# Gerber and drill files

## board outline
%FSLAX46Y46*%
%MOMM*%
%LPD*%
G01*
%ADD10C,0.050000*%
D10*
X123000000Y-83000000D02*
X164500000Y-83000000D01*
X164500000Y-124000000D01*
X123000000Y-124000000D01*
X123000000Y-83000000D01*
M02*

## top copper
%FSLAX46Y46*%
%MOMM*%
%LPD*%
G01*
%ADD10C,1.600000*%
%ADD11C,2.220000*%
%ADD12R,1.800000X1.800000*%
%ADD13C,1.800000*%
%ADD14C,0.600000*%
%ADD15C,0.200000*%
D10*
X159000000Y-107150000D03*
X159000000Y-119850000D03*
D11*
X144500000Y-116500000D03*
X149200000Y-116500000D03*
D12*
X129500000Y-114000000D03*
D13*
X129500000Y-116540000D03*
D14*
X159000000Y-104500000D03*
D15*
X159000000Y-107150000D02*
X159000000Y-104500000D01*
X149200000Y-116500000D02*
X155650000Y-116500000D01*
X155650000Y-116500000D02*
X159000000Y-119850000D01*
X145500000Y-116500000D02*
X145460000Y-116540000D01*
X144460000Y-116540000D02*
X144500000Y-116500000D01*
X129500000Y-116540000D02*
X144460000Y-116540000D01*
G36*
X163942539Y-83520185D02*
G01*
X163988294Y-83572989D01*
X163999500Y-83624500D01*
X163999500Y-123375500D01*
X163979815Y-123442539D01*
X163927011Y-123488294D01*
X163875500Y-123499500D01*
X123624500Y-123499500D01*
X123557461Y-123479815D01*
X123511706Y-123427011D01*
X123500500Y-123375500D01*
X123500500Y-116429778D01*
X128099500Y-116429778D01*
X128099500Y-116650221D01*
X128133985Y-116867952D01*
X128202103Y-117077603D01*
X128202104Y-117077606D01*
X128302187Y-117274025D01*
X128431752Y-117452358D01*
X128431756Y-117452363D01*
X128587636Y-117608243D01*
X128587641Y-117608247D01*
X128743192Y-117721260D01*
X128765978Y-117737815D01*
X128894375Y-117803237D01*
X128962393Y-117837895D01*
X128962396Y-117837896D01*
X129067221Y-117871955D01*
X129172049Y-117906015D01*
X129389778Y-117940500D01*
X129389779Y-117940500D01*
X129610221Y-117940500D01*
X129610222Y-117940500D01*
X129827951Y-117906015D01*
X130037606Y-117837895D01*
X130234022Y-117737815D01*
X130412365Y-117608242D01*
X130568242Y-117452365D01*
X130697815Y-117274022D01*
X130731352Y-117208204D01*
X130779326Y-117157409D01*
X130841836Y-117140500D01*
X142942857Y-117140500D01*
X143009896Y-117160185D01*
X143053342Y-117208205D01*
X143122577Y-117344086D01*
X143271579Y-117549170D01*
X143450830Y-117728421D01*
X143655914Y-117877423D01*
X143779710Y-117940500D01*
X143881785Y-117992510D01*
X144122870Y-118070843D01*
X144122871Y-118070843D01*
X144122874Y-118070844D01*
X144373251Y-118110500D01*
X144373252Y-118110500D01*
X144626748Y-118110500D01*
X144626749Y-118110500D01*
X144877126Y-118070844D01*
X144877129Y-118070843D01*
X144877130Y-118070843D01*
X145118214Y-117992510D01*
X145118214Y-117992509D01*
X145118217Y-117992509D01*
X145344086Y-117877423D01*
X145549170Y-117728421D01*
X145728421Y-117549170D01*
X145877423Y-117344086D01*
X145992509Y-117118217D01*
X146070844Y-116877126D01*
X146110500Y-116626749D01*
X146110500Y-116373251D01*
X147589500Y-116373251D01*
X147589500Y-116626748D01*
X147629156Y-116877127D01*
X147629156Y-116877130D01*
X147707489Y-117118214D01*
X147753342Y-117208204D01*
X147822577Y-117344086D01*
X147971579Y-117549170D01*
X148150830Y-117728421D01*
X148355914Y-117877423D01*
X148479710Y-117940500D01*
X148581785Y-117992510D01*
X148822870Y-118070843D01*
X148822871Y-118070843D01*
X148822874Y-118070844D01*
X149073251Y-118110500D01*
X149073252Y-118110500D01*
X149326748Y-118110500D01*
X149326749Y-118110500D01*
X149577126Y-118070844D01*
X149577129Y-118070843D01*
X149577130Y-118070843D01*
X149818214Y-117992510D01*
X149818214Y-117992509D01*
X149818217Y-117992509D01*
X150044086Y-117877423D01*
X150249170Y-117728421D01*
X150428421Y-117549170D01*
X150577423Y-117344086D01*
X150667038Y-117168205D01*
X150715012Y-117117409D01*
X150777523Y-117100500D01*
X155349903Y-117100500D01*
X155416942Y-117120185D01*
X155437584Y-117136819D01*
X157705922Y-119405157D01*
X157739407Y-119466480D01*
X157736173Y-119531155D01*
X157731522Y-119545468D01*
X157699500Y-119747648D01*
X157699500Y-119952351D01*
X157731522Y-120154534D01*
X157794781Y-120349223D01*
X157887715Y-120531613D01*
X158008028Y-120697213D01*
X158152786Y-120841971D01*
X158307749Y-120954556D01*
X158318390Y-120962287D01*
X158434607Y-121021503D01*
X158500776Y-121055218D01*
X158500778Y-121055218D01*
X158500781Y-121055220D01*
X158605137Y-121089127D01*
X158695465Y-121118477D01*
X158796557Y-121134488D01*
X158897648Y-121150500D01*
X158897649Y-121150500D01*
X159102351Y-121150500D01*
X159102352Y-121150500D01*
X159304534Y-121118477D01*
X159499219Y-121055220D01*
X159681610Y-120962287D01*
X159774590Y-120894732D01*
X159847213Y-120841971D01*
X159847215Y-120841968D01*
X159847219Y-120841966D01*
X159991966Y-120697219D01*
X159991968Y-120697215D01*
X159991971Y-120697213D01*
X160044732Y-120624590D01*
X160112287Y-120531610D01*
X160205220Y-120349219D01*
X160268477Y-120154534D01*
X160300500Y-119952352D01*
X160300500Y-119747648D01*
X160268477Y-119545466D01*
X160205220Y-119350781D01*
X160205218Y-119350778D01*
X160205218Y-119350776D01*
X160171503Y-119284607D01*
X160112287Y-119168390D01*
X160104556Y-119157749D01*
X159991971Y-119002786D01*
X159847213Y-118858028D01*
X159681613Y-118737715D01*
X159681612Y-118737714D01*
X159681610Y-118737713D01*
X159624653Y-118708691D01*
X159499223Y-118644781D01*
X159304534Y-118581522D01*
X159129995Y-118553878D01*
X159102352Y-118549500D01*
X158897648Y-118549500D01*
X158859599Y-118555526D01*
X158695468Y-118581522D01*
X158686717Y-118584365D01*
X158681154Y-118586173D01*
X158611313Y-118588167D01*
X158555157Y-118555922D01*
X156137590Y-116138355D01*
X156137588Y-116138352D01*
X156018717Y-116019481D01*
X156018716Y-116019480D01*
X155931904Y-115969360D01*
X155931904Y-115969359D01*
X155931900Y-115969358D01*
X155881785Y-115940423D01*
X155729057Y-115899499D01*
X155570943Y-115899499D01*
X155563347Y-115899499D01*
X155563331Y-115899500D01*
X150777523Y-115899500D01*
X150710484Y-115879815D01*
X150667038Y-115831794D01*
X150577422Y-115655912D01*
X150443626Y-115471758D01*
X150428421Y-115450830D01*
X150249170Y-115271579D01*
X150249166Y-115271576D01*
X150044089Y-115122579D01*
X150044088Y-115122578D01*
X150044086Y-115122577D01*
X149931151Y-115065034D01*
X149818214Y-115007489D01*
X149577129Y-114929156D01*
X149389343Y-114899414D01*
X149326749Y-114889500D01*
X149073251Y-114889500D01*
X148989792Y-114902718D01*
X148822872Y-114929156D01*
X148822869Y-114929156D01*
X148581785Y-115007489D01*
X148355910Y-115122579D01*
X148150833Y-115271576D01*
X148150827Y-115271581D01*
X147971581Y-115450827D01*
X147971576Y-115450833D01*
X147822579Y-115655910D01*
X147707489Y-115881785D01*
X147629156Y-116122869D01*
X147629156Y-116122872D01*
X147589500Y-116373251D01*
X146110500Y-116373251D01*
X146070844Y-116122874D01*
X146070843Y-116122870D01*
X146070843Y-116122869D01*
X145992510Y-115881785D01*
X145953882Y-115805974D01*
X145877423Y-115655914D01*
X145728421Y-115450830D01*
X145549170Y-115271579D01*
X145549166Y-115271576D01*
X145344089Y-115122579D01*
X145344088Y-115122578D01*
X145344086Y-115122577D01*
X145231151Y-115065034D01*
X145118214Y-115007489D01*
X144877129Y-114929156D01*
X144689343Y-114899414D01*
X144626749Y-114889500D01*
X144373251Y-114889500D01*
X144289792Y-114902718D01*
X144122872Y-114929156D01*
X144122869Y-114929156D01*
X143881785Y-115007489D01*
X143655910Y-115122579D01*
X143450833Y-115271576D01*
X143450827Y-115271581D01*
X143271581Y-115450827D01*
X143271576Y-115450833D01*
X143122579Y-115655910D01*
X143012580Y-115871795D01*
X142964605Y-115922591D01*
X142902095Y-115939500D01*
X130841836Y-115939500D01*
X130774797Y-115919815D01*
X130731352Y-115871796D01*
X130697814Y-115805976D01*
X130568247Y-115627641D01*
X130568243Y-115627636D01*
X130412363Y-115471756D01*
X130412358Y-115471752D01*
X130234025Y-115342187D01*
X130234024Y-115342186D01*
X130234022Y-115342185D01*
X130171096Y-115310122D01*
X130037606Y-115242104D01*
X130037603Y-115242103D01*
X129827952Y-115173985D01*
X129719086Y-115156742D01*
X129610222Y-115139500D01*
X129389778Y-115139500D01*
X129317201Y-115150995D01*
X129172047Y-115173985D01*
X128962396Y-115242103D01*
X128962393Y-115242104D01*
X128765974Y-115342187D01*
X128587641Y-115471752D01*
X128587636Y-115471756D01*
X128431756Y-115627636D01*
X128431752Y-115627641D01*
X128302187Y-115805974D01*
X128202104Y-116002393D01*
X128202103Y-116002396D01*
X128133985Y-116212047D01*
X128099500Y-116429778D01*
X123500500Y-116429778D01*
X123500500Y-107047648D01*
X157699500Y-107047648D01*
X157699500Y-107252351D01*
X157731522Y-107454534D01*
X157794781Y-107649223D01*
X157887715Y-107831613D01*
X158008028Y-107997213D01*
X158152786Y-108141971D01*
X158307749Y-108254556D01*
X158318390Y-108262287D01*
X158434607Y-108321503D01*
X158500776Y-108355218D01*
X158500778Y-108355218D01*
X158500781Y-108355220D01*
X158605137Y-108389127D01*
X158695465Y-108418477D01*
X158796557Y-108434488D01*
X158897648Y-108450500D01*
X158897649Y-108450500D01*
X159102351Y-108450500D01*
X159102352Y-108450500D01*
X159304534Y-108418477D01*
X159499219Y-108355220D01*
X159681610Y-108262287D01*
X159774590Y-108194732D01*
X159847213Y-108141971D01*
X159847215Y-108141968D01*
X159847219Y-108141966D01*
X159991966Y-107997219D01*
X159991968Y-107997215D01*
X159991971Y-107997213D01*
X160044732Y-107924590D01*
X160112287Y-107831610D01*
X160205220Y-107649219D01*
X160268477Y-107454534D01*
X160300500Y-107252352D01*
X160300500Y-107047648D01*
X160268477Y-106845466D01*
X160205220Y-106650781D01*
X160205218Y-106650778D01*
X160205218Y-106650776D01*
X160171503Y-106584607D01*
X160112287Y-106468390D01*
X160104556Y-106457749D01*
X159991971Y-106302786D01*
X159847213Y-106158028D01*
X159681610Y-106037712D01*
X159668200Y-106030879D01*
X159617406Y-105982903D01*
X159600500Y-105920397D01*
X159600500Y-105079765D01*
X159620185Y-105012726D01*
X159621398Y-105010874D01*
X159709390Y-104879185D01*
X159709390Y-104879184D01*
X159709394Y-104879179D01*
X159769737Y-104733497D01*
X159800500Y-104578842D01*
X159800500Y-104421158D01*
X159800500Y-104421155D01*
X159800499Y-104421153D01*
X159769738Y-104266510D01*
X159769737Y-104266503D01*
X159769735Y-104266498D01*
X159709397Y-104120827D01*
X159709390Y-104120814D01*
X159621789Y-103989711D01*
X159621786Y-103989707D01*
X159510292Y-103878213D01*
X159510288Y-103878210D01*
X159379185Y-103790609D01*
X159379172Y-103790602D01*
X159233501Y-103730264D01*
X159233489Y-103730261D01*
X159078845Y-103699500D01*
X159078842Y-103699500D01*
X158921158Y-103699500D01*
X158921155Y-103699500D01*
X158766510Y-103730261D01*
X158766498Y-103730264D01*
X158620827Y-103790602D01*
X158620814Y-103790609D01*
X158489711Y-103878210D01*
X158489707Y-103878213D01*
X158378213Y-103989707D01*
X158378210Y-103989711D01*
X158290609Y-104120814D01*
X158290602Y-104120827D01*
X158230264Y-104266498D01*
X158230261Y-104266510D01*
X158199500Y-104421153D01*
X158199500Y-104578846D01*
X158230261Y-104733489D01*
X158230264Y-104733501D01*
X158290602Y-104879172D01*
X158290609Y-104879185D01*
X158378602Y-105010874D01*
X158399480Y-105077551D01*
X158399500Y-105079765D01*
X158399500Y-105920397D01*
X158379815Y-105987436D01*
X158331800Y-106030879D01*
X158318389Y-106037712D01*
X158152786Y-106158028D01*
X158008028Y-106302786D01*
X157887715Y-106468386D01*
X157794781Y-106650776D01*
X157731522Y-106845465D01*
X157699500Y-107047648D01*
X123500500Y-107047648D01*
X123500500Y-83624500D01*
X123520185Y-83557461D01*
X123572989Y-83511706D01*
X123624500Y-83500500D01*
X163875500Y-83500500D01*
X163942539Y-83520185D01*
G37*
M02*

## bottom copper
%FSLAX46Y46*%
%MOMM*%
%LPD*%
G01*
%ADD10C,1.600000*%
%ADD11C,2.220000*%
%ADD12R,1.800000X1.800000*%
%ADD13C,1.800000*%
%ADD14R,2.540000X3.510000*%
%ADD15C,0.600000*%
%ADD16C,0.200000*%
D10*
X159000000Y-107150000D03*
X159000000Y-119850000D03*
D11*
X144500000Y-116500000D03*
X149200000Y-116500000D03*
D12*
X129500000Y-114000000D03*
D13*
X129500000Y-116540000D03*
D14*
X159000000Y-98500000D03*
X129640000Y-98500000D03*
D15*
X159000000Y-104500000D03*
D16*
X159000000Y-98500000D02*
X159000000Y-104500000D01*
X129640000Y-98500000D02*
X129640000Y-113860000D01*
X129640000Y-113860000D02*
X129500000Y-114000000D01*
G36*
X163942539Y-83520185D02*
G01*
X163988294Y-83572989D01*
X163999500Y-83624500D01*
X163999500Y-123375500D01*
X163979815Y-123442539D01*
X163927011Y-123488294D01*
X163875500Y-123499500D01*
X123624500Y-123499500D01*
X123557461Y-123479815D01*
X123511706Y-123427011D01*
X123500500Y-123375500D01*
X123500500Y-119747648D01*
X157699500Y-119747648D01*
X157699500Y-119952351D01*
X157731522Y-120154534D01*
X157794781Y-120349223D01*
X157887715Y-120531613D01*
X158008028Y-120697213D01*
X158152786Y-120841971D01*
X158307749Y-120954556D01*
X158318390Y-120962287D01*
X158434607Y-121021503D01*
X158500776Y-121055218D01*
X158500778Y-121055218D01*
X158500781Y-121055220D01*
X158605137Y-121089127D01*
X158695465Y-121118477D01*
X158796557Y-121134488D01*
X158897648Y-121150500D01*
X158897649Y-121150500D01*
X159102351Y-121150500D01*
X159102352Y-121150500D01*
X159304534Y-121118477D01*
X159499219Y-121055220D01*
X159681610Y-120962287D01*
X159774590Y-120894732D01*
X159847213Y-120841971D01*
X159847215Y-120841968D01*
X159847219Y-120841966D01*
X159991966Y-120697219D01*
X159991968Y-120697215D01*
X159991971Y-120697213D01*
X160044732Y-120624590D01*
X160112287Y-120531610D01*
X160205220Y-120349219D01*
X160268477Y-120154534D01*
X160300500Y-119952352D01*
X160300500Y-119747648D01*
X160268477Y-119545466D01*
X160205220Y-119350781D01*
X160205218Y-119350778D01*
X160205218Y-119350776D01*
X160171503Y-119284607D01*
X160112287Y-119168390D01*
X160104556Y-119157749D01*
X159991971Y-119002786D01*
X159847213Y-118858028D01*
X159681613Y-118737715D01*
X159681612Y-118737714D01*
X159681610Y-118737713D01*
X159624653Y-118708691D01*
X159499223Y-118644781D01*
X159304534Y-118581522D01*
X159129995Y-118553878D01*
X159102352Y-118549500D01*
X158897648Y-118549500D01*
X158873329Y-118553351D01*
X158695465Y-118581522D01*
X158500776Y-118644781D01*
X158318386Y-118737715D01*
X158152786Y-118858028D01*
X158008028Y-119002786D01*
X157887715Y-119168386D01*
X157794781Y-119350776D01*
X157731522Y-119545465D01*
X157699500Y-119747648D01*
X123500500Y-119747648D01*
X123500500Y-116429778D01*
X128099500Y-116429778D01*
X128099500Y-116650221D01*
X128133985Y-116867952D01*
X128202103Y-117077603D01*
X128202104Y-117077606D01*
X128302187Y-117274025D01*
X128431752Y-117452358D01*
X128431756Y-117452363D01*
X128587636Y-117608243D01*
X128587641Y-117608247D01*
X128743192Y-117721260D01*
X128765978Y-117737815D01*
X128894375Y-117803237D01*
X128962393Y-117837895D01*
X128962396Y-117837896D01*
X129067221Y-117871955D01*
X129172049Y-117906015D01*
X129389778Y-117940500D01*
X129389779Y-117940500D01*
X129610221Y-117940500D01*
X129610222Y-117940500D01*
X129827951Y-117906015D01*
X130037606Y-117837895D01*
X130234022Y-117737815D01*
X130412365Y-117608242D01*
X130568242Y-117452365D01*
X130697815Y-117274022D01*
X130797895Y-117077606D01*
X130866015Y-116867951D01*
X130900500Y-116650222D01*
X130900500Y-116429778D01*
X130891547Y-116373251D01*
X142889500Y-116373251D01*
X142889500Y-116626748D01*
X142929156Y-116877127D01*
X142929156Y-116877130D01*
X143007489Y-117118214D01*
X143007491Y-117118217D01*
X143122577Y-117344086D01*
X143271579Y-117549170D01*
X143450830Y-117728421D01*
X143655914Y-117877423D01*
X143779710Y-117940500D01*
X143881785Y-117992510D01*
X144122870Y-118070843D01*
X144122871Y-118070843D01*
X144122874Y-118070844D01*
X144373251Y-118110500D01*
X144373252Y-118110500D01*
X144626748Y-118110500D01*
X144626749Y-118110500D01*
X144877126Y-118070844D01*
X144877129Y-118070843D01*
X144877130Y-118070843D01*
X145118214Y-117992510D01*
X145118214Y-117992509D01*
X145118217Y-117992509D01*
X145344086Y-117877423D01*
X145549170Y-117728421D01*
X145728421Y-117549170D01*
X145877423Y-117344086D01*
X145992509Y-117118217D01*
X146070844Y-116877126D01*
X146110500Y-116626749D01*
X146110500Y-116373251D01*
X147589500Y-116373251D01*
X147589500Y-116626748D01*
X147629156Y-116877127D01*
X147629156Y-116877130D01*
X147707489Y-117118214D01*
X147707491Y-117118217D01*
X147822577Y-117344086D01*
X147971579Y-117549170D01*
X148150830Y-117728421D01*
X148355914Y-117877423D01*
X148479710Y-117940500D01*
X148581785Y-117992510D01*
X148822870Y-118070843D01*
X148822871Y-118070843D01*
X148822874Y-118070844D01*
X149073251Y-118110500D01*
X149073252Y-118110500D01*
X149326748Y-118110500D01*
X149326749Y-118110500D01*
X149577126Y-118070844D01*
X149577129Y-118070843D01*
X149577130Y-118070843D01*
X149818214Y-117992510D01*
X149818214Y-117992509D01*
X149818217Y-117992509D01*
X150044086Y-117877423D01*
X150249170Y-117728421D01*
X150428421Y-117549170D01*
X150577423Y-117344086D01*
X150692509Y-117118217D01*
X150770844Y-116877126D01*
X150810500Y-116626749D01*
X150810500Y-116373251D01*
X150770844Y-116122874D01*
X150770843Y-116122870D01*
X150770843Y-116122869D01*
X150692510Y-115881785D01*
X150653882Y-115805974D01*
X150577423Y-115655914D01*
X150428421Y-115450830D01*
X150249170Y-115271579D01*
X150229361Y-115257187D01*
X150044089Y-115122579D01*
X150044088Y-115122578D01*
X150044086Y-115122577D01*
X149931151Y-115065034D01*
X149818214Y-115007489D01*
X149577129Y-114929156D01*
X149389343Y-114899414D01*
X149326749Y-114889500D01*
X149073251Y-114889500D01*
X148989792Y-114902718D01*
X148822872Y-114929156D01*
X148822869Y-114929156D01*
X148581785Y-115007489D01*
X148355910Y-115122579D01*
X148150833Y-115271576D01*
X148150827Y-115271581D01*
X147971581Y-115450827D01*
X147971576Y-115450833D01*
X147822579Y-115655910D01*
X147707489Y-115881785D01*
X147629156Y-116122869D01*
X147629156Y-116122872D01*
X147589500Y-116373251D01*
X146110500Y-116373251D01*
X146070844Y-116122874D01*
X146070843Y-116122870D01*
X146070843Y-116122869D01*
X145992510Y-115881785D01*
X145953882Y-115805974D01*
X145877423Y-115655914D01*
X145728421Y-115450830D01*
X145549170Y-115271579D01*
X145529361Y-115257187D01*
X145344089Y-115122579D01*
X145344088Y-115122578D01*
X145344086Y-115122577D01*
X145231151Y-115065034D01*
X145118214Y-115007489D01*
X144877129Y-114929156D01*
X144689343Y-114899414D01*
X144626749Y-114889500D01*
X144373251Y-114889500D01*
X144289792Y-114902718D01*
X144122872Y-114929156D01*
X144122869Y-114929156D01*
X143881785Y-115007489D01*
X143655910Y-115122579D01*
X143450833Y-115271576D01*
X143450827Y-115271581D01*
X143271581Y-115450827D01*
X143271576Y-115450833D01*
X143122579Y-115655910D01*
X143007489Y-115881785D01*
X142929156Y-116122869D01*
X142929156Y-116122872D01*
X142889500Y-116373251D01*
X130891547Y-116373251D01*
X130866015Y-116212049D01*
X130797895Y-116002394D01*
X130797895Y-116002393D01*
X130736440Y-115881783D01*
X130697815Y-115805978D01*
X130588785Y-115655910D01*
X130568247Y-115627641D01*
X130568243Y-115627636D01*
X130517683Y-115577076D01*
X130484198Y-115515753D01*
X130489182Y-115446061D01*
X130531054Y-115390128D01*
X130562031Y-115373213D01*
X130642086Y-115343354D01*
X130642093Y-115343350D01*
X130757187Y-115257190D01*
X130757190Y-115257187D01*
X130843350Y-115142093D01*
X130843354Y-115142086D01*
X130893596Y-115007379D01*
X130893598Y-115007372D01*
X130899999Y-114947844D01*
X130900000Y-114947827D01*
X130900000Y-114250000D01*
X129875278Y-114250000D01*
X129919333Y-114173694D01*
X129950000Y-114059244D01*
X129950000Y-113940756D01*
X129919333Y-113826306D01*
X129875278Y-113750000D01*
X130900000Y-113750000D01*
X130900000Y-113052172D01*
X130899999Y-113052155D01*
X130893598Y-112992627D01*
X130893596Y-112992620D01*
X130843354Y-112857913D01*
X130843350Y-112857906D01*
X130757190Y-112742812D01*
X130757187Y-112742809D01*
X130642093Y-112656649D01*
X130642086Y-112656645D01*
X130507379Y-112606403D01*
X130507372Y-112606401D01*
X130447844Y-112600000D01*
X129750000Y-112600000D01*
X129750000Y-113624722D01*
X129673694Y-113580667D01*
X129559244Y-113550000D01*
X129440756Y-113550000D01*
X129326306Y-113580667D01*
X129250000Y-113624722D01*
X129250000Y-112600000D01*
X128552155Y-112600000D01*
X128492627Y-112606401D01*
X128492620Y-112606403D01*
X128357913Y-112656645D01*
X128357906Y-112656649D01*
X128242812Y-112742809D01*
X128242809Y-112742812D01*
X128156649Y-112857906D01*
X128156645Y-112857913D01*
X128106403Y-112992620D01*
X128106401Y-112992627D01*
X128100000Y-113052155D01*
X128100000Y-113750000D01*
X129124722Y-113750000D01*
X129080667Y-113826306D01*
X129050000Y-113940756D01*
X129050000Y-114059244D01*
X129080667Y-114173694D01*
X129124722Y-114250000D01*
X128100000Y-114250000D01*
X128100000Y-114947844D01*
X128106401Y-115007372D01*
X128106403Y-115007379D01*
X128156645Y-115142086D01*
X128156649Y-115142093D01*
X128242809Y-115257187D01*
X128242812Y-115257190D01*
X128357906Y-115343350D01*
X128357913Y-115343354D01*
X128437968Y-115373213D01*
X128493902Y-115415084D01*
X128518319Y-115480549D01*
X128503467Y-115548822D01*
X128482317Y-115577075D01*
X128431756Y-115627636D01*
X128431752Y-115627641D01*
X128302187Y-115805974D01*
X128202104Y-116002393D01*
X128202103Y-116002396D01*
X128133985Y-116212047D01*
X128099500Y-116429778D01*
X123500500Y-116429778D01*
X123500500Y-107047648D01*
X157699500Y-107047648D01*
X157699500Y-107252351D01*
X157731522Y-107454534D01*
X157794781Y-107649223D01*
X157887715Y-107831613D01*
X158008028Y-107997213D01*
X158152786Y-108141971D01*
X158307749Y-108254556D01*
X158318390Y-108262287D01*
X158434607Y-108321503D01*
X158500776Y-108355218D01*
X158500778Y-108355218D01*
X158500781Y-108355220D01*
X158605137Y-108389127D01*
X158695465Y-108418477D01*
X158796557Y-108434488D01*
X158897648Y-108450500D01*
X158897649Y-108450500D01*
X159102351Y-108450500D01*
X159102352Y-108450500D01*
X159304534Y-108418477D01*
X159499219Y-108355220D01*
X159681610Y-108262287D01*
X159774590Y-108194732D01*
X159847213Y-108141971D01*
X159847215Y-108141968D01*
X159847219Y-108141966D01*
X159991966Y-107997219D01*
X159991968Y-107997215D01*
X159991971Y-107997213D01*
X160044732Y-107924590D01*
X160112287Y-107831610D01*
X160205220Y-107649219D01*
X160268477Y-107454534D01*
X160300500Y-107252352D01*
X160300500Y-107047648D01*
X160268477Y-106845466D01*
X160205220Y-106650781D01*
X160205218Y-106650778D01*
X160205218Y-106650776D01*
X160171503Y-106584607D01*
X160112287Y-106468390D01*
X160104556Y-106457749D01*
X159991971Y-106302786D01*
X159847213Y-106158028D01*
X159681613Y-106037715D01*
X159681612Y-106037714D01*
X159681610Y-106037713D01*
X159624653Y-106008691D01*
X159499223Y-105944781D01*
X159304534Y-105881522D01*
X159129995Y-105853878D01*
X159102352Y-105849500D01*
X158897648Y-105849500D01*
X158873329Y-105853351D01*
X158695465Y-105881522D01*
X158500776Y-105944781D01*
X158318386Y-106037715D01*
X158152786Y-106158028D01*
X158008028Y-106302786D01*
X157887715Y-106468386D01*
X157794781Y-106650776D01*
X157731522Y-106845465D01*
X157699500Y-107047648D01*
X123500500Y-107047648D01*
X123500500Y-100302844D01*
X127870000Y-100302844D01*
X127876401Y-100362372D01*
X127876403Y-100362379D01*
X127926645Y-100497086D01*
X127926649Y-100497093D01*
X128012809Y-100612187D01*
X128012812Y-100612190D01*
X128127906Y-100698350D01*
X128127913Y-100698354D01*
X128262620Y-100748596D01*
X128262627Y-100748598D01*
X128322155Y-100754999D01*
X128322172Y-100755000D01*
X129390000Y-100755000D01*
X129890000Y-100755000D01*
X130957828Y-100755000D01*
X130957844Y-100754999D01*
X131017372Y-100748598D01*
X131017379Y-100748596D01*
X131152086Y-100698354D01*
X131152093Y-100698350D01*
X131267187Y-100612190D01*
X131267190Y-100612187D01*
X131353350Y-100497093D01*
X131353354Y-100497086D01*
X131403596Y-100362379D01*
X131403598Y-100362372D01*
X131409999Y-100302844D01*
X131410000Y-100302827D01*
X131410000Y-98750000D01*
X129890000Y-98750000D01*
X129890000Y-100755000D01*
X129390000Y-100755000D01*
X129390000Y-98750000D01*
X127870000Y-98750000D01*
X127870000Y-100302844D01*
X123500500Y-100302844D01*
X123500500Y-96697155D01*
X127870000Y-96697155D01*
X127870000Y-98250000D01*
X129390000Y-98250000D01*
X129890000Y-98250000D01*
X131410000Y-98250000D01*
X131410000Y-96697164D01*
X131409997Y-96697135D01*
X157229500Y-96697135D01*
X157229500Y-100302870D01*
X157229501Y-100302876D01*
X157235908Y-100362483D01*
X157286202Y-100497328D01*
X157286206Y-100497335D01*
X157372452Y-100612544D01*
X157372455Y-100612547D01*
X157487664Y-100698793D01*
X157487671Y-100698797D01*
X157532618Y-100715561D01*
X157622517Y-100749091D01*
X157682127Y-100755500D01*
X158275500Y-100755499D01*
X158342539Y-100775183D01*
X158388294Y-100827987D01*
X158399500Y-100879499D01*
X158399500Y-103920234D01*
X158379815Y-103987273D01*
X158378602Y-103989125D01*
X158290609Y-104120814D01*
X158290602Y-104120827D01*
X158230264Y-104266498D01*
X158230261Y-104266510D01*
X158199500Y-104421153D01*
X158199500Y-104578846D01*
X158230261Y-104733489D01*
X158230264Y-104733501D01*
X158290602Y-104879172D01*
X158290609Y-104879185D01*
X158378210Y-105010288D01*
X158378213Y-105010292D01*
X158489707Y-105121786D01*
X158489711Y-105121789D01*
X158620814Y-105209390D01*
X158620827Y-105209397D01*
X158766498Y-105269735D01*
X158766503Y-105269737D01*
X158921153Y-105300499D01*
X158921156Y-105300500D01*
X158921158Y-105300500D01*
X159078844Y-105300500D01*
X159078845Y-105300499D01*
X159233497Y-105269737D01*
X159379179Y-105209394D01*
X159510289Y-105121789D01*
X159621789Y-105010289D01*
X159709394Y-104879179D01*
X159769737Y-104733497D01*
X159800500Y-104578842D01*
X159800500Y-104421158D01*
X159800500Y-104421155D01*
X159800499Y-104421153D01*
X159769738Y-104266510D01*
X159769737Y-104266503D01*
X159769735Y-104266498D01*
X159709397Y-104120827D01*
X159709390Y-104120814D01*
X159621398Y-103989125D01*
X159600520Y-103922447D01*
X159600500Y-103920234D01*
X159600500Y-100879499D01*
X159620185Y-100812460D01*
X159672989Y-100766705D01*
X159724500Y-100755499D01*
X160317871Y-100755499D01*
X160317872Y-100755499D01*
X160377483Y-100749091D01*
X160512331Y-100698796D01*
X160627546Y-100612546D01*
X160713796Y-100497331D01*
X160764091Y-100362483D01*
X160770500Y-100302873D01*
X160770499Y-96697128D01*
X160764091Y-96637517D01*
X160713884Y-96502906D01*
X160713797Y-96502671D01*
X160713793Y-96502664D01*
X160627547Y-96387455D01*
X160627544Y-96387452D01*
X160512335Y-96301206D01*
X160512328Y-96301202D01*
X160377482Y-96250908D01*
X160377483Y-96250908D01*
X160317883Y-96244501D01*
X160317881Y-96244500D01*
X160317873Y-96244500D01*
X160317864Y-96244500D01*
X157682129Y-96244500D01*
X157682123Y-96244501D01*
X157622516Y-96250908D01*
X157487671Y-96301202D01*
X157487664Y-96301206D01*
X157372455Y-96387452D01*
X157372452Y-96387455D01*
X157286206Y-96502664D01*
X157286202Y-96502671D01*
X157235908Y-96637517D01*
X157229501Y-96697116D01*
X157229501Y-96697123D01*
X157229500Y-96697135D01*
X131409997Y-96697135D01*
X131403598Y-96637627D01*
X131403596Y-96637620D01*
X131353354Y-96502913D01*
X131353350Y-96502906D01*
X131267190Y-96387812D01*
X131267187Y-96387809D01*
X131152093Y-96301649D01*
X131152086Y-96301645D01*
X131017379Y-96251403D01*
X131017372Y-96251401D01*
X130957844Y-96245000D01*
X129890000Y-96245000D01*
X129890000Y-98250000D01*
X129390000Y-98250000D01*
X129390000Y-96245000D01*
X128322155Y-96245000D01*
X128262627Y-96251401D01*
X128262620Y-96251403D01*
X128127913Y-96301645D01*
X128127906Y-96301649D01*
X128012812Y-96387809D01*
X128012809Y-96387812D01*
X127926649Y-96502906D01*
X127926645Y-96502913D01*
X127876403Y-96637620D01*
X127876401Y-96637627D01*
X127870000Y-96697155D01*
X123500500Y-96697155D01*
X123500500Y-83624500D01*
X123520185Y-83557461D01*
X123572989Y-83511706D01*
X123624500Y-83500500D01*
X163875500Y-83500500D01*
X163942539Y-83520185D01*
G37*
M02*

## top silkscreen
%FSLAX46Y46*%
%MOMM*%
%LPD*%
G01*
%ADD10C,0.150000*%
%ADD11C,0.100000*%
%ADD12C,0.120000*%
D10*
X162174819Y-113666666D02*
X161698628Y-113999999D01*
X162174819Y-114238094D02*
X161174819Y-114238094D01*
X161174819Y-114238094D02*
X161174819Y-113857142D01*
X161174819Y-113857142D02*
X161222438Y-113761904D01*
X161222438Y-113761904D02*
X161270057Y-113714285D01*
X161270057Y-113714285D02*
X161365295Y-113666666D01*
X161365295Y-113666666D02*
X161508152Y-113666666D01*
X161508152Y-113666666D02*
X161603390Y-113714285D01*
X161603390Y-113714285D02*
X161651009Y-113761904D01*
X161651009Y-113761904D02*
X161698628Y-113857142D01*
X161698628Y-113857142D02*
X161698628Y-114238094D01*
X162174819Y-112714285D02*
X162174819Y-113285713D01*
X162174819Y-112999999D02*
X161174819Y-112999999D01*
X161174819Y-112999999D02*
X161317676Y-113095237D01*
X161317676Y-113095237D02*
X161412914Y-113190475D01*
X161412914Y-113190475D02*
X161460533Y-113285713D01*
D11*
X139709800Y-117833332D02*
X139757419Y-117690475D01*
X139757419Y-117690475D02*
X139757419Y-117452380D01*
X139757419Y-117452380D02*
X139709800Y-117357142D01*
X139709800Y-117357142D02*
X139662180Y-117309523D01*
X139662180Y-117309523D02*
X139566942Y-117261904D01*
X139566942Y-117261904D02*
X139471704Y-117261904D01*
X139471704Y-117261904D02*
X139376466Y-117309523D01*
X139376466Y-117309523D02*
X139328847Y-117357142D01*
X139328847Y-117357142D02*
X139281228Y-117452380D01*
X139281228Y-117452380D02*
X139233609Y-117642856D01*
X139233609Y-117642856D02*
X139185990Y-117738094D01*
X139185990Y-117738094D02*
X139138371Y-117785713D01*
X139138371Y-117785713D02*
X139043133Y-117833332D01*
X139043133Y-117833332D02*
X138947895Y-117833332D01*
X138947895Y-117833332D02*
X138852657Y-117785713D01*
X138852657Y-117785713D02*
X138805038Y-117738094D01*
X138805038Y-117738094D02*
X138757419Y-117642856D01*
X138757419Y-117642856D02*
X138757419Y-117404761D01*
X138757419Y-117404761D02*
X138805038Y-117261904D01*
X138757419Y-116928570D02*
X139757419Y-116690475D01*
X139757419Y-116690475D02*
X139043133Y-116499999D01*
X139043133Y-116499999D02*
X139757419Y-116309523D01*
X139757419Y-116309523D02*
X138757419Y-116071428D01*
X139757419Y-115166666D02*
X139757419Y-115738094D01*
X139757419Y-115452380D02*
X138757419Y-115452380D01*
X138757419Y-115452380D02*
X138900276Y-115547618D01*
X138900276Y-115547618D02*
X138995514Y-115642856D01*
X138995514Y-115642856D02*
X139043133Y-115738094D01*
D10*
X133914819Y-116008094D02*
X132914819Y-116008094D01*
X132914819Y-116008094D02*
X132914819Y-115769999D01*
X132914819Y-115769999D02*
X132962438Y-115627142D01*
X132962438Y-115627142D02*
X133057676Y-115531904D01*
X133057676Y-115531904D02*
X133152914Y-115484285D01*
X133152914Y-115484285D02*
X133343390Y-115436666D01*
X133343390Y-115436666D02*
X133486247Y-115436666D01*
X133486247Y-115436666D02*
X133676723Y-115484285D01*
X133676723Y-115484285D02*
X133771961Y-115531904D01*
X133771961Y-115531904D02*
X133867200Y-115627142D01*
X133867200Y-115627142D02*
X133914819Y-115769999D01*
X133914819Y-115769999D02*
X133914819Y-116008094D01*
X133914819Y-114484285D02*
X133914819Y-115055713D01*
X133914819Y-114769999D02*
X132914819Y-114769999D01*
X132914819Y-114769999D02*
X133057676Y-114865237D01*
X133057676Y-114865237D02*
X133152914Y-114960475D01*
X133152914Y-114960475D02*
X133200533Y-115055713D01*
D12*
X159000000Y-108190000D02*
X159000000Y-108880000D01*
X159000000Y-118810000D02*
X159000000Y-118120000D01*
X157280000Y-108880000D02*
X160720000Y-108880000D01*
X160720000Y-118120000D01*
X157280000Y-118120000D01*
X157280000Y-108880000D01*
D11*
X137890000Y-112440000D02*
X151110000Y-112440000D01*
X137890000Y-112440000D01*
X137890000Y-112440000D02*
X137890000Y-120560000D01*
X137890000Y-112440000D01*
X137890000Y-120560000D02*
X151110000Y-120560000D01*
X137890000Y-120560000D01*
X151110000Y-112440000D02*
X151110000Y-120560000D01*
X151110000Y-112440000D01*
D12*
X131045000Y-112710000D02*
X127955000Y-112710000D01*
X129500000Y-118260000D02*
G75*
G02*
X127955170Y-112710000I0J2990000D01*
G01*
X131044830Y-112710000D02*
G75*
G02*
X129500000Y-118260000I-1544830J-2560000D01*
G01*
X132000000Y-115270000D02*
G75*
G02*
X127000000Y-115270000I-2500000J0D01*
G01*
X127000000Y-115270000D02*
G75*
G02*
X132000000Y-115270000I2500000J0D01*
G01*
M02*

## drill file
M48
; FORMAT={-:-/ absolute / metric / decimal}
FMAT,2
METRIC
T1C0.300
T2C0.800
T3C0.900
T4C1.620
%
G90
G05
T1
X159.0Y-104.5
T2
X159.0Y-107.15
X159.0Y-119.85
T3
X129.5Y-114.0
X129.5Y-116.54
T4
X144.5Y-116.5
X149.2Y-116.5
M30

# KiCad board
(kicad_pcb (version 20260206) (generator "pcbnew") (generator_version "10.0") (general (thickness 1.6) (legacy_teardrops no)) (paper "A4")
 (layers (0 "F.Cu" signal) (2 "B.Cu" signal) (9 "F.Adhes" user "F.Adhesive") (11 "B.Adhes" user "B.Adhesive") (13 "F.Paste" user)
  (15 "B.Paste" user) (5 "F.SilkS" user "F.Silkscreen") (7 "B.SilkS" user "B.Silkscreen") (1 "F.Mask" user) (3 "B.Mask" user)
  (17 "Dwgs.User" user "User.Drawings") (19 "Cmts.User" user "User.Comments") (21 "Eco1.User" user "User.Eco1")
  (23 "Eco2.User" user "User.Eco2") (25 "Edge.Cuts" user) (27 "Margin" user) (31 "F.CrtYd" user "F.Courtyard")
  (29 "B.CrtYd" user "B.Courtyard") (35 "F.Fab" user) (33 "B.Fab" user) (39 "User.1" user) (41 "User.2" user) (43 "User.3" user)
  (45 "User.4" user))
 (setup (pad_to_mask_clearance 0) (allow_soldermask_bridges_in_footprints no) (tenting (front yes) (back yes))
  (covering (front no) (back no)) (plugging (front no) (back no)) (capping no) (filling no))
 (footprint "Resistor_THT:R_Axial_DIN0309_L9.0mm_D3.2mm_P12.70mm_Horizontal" (layer "F.Cu") (at 159 107.15 -90)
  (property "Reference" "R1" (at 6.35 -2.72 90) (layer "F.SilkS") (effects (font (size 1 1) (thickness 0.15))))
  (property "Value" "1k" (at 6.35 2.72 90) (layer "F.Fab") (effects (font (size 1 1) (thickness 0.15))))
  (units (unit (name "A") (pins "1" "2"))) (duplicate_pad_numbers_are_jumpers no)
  (fp_line (start 1.04 0) (end 1.73 0) (stroke (width 0.12) (type solid)) (layer "F.SilkS"))
  (fp_line (start 11.66 0) (end 10.97 0) (stroke (width 0.12) (type solid)) (layer "F.SilkS"))
  (fp_rect (start 1.73 -1.72) (end 10.97 1.72) (stroke (width 0.12) (type solid)) (fill no) (layer "F.SilkS"))
  (pad "1" thru_hole circle (at 0 0 270) (size 1.6 1.6) (drill 0.8) (layers "*.Cu" "*.Mask") (remove_unused_layers no) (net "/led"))
  (pad "2" thru_hole circle (at 12.7 0 270) (size 1.6 1.6) (drill 0.8) (layers "*.Cu" "*.Mask") (remove_unused_layers no) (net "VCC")))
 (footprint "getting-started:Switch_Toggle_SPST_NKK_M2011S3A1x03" (layer "F.Cu") (at 139.8 116.5 90)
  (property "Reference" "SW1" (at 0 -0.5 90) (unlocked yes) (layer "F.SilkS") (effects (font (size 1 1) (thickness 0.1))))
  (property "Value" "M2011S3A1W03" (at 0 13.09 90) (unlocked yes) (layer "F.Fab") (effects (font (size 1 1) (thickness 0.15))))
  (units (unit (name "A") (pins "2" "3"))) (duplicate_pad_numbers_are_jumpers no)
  (fp_rect (start 4.06 -1.91) (end 4.06 11.31) (stroke (width 0.1) (type default)) (fill no) (layer "F.SilkS"))
  (fp_rect (start -4.06 -1.91) (end 4.06 -1.91) (stroke (width 0.1) (type default)) (fill no) (layer "F.SilkS"))
  (fp_rect (start -4.06 -1.91) (end -4.06 11.31) (stroke (width 0.1) (type default)) (fill no) (layer "F.SilkS"))
  (fp_rect (start -4.06 11.31) (end 4.06 11.31) (stroke (width 0.1) (type default)) (fill no) (layer "F.SilkS"))
  (pad "2" thru_hole circle (at 0 4.7 90) (size 2.22 2.22) (drill 1.62) (layers "*.Cu" "*.Mask") (remove_unused_layers no)
   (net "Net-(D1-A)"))
  (pad "3" thru_hole circle (at 0 9.4 90) (size 2.22 2.22) (drill 1.62) (layers "*.Cu" "*.Mask") (remove_unused_layers no) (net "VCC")))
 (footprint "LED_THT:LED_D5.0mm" (layer "F.Cu") (at 129.5 114 -90)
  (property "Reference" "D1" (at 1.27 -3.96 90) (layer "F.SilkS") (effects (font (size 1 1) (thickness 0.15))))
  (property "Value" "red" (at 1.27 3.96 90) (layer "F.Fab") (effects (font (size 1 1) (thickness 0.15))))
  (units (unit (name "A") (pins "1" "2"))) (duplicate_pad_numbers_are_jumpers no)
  (fp_line (start -1.29 -1.545) (end -1.29 1.545) (stroke (width 0.12) (type solid)) (layer "F.SilkS"))
  (fp_arc (start 4.26 0) (mid 2.071779 2.880495) (end -1.29 1.54483) (stroke (width 0.12) (type solid)) (layer "F.SilkS"))
  (fp_arc (start -1.29 -1.54483) (mid 2.071779 -2.880495) (end 4.26 0) (stroke (width 0.12) (type solid)) (layer "F.SilkS"))
  (fp_circle (center 1.27 0) (end 3.77 0) (stroke (width 0.12) (type solid)) (fill no) (layer "F.SilkS"))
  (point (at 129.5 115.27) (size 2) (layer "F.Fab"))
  (pad "1" thru_hole rect (at 0 0 270) (size 1.8 1.8) (drill 0.9) (layers "*.Cu" "*.Mask") (remove_unused_layers no) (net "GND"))
  (pad "2" thru_hole circle (at 2.54 0 270) (size 1.8 1.8) (drill 0.9) (layers "*.Cu" "*.Mask") (remove_unused_layers no) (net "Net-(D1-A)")))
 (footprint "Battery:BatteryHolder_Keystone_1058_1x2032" (layer "B.Cu") (at 144.32 98.5 180)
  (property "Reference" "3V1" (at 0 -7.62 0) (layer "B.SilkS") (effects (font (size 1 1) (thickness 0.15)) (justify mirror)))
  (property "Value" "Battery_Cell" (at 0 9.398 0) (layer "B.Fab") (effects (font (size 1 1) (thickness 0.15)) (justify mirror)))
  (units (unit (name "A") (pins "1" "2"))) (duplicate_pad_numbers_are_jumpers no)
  (pad "1" smd rect (at -14.68 0 180) (size 2.54 3.51) (layers "B.Cu" "B.Mask" "B.Paste") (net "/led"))
  (pad "2" smd rect (at 14.68 0 180) (size 2.54 3.51) (layers "B.Cu" "B.Mask" "B.Paste") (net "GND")))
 (gr_rect (start 123 83) (end 164.5 124) (stroke (width 0.05) (type default)) (fill no) (layer "Edge.Cuts"))
 (segment (start 159 107.15) (end 159 104.5) (width 0.2) (layer "F.Cu") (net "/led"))
 (via (at 159 104.5) (size 0.6) (drill 0.3) (layers "F.Cu" "B.Cu") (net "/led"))
 (segment (start 159 98.5) (end 159 104.5) (width 0.2) (layer "B.Cu") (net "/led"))
 (segment (start 149.2 116.5) (end 155.65 116.5) (width 0.2) (layer "F.Cu") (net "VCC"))
 (segment (start 155.65 116.5) (end 159 119.85) (width 0.2) (layer "F.Cu") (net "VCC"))
 (segment (start 129.64 98.5) (end 129.64 113.86) (width 0.2) (layer "B.Cu") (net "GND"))
 (segment (start 129.64 113.86) (end 129.5 114) (width 0.2) (layer "B.Cu") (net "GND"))
 (segment (start 145.5 116.5) (end 145.46 116.54) (width 0.2) (layer "F.Cu") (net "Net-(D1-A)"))
 (segment (start 144.46 116.54) (end 144.5 116.5) (width 0.2) (layer "F.Cu") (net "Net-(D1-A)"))
 (segment (start 129.5 116.54) (end 144.46 116.54) (width 0.2) (layer "F.Cu") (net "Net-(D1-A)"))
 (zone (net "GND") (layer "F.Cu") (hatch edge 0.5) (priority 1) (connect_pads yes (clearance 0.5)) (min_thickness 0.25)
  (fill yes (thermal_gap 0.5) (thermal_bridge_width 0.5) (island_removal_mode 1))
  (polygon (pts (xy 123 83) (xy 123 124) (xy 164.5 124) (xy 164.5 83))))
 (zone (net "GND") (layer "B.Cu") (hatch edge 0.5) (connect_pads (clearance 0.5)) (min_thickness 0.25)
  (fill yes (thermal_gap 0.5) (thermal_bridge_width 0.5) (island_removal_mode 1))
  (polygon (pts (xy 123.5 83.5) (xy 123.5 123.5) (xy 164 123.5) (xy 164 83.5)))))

